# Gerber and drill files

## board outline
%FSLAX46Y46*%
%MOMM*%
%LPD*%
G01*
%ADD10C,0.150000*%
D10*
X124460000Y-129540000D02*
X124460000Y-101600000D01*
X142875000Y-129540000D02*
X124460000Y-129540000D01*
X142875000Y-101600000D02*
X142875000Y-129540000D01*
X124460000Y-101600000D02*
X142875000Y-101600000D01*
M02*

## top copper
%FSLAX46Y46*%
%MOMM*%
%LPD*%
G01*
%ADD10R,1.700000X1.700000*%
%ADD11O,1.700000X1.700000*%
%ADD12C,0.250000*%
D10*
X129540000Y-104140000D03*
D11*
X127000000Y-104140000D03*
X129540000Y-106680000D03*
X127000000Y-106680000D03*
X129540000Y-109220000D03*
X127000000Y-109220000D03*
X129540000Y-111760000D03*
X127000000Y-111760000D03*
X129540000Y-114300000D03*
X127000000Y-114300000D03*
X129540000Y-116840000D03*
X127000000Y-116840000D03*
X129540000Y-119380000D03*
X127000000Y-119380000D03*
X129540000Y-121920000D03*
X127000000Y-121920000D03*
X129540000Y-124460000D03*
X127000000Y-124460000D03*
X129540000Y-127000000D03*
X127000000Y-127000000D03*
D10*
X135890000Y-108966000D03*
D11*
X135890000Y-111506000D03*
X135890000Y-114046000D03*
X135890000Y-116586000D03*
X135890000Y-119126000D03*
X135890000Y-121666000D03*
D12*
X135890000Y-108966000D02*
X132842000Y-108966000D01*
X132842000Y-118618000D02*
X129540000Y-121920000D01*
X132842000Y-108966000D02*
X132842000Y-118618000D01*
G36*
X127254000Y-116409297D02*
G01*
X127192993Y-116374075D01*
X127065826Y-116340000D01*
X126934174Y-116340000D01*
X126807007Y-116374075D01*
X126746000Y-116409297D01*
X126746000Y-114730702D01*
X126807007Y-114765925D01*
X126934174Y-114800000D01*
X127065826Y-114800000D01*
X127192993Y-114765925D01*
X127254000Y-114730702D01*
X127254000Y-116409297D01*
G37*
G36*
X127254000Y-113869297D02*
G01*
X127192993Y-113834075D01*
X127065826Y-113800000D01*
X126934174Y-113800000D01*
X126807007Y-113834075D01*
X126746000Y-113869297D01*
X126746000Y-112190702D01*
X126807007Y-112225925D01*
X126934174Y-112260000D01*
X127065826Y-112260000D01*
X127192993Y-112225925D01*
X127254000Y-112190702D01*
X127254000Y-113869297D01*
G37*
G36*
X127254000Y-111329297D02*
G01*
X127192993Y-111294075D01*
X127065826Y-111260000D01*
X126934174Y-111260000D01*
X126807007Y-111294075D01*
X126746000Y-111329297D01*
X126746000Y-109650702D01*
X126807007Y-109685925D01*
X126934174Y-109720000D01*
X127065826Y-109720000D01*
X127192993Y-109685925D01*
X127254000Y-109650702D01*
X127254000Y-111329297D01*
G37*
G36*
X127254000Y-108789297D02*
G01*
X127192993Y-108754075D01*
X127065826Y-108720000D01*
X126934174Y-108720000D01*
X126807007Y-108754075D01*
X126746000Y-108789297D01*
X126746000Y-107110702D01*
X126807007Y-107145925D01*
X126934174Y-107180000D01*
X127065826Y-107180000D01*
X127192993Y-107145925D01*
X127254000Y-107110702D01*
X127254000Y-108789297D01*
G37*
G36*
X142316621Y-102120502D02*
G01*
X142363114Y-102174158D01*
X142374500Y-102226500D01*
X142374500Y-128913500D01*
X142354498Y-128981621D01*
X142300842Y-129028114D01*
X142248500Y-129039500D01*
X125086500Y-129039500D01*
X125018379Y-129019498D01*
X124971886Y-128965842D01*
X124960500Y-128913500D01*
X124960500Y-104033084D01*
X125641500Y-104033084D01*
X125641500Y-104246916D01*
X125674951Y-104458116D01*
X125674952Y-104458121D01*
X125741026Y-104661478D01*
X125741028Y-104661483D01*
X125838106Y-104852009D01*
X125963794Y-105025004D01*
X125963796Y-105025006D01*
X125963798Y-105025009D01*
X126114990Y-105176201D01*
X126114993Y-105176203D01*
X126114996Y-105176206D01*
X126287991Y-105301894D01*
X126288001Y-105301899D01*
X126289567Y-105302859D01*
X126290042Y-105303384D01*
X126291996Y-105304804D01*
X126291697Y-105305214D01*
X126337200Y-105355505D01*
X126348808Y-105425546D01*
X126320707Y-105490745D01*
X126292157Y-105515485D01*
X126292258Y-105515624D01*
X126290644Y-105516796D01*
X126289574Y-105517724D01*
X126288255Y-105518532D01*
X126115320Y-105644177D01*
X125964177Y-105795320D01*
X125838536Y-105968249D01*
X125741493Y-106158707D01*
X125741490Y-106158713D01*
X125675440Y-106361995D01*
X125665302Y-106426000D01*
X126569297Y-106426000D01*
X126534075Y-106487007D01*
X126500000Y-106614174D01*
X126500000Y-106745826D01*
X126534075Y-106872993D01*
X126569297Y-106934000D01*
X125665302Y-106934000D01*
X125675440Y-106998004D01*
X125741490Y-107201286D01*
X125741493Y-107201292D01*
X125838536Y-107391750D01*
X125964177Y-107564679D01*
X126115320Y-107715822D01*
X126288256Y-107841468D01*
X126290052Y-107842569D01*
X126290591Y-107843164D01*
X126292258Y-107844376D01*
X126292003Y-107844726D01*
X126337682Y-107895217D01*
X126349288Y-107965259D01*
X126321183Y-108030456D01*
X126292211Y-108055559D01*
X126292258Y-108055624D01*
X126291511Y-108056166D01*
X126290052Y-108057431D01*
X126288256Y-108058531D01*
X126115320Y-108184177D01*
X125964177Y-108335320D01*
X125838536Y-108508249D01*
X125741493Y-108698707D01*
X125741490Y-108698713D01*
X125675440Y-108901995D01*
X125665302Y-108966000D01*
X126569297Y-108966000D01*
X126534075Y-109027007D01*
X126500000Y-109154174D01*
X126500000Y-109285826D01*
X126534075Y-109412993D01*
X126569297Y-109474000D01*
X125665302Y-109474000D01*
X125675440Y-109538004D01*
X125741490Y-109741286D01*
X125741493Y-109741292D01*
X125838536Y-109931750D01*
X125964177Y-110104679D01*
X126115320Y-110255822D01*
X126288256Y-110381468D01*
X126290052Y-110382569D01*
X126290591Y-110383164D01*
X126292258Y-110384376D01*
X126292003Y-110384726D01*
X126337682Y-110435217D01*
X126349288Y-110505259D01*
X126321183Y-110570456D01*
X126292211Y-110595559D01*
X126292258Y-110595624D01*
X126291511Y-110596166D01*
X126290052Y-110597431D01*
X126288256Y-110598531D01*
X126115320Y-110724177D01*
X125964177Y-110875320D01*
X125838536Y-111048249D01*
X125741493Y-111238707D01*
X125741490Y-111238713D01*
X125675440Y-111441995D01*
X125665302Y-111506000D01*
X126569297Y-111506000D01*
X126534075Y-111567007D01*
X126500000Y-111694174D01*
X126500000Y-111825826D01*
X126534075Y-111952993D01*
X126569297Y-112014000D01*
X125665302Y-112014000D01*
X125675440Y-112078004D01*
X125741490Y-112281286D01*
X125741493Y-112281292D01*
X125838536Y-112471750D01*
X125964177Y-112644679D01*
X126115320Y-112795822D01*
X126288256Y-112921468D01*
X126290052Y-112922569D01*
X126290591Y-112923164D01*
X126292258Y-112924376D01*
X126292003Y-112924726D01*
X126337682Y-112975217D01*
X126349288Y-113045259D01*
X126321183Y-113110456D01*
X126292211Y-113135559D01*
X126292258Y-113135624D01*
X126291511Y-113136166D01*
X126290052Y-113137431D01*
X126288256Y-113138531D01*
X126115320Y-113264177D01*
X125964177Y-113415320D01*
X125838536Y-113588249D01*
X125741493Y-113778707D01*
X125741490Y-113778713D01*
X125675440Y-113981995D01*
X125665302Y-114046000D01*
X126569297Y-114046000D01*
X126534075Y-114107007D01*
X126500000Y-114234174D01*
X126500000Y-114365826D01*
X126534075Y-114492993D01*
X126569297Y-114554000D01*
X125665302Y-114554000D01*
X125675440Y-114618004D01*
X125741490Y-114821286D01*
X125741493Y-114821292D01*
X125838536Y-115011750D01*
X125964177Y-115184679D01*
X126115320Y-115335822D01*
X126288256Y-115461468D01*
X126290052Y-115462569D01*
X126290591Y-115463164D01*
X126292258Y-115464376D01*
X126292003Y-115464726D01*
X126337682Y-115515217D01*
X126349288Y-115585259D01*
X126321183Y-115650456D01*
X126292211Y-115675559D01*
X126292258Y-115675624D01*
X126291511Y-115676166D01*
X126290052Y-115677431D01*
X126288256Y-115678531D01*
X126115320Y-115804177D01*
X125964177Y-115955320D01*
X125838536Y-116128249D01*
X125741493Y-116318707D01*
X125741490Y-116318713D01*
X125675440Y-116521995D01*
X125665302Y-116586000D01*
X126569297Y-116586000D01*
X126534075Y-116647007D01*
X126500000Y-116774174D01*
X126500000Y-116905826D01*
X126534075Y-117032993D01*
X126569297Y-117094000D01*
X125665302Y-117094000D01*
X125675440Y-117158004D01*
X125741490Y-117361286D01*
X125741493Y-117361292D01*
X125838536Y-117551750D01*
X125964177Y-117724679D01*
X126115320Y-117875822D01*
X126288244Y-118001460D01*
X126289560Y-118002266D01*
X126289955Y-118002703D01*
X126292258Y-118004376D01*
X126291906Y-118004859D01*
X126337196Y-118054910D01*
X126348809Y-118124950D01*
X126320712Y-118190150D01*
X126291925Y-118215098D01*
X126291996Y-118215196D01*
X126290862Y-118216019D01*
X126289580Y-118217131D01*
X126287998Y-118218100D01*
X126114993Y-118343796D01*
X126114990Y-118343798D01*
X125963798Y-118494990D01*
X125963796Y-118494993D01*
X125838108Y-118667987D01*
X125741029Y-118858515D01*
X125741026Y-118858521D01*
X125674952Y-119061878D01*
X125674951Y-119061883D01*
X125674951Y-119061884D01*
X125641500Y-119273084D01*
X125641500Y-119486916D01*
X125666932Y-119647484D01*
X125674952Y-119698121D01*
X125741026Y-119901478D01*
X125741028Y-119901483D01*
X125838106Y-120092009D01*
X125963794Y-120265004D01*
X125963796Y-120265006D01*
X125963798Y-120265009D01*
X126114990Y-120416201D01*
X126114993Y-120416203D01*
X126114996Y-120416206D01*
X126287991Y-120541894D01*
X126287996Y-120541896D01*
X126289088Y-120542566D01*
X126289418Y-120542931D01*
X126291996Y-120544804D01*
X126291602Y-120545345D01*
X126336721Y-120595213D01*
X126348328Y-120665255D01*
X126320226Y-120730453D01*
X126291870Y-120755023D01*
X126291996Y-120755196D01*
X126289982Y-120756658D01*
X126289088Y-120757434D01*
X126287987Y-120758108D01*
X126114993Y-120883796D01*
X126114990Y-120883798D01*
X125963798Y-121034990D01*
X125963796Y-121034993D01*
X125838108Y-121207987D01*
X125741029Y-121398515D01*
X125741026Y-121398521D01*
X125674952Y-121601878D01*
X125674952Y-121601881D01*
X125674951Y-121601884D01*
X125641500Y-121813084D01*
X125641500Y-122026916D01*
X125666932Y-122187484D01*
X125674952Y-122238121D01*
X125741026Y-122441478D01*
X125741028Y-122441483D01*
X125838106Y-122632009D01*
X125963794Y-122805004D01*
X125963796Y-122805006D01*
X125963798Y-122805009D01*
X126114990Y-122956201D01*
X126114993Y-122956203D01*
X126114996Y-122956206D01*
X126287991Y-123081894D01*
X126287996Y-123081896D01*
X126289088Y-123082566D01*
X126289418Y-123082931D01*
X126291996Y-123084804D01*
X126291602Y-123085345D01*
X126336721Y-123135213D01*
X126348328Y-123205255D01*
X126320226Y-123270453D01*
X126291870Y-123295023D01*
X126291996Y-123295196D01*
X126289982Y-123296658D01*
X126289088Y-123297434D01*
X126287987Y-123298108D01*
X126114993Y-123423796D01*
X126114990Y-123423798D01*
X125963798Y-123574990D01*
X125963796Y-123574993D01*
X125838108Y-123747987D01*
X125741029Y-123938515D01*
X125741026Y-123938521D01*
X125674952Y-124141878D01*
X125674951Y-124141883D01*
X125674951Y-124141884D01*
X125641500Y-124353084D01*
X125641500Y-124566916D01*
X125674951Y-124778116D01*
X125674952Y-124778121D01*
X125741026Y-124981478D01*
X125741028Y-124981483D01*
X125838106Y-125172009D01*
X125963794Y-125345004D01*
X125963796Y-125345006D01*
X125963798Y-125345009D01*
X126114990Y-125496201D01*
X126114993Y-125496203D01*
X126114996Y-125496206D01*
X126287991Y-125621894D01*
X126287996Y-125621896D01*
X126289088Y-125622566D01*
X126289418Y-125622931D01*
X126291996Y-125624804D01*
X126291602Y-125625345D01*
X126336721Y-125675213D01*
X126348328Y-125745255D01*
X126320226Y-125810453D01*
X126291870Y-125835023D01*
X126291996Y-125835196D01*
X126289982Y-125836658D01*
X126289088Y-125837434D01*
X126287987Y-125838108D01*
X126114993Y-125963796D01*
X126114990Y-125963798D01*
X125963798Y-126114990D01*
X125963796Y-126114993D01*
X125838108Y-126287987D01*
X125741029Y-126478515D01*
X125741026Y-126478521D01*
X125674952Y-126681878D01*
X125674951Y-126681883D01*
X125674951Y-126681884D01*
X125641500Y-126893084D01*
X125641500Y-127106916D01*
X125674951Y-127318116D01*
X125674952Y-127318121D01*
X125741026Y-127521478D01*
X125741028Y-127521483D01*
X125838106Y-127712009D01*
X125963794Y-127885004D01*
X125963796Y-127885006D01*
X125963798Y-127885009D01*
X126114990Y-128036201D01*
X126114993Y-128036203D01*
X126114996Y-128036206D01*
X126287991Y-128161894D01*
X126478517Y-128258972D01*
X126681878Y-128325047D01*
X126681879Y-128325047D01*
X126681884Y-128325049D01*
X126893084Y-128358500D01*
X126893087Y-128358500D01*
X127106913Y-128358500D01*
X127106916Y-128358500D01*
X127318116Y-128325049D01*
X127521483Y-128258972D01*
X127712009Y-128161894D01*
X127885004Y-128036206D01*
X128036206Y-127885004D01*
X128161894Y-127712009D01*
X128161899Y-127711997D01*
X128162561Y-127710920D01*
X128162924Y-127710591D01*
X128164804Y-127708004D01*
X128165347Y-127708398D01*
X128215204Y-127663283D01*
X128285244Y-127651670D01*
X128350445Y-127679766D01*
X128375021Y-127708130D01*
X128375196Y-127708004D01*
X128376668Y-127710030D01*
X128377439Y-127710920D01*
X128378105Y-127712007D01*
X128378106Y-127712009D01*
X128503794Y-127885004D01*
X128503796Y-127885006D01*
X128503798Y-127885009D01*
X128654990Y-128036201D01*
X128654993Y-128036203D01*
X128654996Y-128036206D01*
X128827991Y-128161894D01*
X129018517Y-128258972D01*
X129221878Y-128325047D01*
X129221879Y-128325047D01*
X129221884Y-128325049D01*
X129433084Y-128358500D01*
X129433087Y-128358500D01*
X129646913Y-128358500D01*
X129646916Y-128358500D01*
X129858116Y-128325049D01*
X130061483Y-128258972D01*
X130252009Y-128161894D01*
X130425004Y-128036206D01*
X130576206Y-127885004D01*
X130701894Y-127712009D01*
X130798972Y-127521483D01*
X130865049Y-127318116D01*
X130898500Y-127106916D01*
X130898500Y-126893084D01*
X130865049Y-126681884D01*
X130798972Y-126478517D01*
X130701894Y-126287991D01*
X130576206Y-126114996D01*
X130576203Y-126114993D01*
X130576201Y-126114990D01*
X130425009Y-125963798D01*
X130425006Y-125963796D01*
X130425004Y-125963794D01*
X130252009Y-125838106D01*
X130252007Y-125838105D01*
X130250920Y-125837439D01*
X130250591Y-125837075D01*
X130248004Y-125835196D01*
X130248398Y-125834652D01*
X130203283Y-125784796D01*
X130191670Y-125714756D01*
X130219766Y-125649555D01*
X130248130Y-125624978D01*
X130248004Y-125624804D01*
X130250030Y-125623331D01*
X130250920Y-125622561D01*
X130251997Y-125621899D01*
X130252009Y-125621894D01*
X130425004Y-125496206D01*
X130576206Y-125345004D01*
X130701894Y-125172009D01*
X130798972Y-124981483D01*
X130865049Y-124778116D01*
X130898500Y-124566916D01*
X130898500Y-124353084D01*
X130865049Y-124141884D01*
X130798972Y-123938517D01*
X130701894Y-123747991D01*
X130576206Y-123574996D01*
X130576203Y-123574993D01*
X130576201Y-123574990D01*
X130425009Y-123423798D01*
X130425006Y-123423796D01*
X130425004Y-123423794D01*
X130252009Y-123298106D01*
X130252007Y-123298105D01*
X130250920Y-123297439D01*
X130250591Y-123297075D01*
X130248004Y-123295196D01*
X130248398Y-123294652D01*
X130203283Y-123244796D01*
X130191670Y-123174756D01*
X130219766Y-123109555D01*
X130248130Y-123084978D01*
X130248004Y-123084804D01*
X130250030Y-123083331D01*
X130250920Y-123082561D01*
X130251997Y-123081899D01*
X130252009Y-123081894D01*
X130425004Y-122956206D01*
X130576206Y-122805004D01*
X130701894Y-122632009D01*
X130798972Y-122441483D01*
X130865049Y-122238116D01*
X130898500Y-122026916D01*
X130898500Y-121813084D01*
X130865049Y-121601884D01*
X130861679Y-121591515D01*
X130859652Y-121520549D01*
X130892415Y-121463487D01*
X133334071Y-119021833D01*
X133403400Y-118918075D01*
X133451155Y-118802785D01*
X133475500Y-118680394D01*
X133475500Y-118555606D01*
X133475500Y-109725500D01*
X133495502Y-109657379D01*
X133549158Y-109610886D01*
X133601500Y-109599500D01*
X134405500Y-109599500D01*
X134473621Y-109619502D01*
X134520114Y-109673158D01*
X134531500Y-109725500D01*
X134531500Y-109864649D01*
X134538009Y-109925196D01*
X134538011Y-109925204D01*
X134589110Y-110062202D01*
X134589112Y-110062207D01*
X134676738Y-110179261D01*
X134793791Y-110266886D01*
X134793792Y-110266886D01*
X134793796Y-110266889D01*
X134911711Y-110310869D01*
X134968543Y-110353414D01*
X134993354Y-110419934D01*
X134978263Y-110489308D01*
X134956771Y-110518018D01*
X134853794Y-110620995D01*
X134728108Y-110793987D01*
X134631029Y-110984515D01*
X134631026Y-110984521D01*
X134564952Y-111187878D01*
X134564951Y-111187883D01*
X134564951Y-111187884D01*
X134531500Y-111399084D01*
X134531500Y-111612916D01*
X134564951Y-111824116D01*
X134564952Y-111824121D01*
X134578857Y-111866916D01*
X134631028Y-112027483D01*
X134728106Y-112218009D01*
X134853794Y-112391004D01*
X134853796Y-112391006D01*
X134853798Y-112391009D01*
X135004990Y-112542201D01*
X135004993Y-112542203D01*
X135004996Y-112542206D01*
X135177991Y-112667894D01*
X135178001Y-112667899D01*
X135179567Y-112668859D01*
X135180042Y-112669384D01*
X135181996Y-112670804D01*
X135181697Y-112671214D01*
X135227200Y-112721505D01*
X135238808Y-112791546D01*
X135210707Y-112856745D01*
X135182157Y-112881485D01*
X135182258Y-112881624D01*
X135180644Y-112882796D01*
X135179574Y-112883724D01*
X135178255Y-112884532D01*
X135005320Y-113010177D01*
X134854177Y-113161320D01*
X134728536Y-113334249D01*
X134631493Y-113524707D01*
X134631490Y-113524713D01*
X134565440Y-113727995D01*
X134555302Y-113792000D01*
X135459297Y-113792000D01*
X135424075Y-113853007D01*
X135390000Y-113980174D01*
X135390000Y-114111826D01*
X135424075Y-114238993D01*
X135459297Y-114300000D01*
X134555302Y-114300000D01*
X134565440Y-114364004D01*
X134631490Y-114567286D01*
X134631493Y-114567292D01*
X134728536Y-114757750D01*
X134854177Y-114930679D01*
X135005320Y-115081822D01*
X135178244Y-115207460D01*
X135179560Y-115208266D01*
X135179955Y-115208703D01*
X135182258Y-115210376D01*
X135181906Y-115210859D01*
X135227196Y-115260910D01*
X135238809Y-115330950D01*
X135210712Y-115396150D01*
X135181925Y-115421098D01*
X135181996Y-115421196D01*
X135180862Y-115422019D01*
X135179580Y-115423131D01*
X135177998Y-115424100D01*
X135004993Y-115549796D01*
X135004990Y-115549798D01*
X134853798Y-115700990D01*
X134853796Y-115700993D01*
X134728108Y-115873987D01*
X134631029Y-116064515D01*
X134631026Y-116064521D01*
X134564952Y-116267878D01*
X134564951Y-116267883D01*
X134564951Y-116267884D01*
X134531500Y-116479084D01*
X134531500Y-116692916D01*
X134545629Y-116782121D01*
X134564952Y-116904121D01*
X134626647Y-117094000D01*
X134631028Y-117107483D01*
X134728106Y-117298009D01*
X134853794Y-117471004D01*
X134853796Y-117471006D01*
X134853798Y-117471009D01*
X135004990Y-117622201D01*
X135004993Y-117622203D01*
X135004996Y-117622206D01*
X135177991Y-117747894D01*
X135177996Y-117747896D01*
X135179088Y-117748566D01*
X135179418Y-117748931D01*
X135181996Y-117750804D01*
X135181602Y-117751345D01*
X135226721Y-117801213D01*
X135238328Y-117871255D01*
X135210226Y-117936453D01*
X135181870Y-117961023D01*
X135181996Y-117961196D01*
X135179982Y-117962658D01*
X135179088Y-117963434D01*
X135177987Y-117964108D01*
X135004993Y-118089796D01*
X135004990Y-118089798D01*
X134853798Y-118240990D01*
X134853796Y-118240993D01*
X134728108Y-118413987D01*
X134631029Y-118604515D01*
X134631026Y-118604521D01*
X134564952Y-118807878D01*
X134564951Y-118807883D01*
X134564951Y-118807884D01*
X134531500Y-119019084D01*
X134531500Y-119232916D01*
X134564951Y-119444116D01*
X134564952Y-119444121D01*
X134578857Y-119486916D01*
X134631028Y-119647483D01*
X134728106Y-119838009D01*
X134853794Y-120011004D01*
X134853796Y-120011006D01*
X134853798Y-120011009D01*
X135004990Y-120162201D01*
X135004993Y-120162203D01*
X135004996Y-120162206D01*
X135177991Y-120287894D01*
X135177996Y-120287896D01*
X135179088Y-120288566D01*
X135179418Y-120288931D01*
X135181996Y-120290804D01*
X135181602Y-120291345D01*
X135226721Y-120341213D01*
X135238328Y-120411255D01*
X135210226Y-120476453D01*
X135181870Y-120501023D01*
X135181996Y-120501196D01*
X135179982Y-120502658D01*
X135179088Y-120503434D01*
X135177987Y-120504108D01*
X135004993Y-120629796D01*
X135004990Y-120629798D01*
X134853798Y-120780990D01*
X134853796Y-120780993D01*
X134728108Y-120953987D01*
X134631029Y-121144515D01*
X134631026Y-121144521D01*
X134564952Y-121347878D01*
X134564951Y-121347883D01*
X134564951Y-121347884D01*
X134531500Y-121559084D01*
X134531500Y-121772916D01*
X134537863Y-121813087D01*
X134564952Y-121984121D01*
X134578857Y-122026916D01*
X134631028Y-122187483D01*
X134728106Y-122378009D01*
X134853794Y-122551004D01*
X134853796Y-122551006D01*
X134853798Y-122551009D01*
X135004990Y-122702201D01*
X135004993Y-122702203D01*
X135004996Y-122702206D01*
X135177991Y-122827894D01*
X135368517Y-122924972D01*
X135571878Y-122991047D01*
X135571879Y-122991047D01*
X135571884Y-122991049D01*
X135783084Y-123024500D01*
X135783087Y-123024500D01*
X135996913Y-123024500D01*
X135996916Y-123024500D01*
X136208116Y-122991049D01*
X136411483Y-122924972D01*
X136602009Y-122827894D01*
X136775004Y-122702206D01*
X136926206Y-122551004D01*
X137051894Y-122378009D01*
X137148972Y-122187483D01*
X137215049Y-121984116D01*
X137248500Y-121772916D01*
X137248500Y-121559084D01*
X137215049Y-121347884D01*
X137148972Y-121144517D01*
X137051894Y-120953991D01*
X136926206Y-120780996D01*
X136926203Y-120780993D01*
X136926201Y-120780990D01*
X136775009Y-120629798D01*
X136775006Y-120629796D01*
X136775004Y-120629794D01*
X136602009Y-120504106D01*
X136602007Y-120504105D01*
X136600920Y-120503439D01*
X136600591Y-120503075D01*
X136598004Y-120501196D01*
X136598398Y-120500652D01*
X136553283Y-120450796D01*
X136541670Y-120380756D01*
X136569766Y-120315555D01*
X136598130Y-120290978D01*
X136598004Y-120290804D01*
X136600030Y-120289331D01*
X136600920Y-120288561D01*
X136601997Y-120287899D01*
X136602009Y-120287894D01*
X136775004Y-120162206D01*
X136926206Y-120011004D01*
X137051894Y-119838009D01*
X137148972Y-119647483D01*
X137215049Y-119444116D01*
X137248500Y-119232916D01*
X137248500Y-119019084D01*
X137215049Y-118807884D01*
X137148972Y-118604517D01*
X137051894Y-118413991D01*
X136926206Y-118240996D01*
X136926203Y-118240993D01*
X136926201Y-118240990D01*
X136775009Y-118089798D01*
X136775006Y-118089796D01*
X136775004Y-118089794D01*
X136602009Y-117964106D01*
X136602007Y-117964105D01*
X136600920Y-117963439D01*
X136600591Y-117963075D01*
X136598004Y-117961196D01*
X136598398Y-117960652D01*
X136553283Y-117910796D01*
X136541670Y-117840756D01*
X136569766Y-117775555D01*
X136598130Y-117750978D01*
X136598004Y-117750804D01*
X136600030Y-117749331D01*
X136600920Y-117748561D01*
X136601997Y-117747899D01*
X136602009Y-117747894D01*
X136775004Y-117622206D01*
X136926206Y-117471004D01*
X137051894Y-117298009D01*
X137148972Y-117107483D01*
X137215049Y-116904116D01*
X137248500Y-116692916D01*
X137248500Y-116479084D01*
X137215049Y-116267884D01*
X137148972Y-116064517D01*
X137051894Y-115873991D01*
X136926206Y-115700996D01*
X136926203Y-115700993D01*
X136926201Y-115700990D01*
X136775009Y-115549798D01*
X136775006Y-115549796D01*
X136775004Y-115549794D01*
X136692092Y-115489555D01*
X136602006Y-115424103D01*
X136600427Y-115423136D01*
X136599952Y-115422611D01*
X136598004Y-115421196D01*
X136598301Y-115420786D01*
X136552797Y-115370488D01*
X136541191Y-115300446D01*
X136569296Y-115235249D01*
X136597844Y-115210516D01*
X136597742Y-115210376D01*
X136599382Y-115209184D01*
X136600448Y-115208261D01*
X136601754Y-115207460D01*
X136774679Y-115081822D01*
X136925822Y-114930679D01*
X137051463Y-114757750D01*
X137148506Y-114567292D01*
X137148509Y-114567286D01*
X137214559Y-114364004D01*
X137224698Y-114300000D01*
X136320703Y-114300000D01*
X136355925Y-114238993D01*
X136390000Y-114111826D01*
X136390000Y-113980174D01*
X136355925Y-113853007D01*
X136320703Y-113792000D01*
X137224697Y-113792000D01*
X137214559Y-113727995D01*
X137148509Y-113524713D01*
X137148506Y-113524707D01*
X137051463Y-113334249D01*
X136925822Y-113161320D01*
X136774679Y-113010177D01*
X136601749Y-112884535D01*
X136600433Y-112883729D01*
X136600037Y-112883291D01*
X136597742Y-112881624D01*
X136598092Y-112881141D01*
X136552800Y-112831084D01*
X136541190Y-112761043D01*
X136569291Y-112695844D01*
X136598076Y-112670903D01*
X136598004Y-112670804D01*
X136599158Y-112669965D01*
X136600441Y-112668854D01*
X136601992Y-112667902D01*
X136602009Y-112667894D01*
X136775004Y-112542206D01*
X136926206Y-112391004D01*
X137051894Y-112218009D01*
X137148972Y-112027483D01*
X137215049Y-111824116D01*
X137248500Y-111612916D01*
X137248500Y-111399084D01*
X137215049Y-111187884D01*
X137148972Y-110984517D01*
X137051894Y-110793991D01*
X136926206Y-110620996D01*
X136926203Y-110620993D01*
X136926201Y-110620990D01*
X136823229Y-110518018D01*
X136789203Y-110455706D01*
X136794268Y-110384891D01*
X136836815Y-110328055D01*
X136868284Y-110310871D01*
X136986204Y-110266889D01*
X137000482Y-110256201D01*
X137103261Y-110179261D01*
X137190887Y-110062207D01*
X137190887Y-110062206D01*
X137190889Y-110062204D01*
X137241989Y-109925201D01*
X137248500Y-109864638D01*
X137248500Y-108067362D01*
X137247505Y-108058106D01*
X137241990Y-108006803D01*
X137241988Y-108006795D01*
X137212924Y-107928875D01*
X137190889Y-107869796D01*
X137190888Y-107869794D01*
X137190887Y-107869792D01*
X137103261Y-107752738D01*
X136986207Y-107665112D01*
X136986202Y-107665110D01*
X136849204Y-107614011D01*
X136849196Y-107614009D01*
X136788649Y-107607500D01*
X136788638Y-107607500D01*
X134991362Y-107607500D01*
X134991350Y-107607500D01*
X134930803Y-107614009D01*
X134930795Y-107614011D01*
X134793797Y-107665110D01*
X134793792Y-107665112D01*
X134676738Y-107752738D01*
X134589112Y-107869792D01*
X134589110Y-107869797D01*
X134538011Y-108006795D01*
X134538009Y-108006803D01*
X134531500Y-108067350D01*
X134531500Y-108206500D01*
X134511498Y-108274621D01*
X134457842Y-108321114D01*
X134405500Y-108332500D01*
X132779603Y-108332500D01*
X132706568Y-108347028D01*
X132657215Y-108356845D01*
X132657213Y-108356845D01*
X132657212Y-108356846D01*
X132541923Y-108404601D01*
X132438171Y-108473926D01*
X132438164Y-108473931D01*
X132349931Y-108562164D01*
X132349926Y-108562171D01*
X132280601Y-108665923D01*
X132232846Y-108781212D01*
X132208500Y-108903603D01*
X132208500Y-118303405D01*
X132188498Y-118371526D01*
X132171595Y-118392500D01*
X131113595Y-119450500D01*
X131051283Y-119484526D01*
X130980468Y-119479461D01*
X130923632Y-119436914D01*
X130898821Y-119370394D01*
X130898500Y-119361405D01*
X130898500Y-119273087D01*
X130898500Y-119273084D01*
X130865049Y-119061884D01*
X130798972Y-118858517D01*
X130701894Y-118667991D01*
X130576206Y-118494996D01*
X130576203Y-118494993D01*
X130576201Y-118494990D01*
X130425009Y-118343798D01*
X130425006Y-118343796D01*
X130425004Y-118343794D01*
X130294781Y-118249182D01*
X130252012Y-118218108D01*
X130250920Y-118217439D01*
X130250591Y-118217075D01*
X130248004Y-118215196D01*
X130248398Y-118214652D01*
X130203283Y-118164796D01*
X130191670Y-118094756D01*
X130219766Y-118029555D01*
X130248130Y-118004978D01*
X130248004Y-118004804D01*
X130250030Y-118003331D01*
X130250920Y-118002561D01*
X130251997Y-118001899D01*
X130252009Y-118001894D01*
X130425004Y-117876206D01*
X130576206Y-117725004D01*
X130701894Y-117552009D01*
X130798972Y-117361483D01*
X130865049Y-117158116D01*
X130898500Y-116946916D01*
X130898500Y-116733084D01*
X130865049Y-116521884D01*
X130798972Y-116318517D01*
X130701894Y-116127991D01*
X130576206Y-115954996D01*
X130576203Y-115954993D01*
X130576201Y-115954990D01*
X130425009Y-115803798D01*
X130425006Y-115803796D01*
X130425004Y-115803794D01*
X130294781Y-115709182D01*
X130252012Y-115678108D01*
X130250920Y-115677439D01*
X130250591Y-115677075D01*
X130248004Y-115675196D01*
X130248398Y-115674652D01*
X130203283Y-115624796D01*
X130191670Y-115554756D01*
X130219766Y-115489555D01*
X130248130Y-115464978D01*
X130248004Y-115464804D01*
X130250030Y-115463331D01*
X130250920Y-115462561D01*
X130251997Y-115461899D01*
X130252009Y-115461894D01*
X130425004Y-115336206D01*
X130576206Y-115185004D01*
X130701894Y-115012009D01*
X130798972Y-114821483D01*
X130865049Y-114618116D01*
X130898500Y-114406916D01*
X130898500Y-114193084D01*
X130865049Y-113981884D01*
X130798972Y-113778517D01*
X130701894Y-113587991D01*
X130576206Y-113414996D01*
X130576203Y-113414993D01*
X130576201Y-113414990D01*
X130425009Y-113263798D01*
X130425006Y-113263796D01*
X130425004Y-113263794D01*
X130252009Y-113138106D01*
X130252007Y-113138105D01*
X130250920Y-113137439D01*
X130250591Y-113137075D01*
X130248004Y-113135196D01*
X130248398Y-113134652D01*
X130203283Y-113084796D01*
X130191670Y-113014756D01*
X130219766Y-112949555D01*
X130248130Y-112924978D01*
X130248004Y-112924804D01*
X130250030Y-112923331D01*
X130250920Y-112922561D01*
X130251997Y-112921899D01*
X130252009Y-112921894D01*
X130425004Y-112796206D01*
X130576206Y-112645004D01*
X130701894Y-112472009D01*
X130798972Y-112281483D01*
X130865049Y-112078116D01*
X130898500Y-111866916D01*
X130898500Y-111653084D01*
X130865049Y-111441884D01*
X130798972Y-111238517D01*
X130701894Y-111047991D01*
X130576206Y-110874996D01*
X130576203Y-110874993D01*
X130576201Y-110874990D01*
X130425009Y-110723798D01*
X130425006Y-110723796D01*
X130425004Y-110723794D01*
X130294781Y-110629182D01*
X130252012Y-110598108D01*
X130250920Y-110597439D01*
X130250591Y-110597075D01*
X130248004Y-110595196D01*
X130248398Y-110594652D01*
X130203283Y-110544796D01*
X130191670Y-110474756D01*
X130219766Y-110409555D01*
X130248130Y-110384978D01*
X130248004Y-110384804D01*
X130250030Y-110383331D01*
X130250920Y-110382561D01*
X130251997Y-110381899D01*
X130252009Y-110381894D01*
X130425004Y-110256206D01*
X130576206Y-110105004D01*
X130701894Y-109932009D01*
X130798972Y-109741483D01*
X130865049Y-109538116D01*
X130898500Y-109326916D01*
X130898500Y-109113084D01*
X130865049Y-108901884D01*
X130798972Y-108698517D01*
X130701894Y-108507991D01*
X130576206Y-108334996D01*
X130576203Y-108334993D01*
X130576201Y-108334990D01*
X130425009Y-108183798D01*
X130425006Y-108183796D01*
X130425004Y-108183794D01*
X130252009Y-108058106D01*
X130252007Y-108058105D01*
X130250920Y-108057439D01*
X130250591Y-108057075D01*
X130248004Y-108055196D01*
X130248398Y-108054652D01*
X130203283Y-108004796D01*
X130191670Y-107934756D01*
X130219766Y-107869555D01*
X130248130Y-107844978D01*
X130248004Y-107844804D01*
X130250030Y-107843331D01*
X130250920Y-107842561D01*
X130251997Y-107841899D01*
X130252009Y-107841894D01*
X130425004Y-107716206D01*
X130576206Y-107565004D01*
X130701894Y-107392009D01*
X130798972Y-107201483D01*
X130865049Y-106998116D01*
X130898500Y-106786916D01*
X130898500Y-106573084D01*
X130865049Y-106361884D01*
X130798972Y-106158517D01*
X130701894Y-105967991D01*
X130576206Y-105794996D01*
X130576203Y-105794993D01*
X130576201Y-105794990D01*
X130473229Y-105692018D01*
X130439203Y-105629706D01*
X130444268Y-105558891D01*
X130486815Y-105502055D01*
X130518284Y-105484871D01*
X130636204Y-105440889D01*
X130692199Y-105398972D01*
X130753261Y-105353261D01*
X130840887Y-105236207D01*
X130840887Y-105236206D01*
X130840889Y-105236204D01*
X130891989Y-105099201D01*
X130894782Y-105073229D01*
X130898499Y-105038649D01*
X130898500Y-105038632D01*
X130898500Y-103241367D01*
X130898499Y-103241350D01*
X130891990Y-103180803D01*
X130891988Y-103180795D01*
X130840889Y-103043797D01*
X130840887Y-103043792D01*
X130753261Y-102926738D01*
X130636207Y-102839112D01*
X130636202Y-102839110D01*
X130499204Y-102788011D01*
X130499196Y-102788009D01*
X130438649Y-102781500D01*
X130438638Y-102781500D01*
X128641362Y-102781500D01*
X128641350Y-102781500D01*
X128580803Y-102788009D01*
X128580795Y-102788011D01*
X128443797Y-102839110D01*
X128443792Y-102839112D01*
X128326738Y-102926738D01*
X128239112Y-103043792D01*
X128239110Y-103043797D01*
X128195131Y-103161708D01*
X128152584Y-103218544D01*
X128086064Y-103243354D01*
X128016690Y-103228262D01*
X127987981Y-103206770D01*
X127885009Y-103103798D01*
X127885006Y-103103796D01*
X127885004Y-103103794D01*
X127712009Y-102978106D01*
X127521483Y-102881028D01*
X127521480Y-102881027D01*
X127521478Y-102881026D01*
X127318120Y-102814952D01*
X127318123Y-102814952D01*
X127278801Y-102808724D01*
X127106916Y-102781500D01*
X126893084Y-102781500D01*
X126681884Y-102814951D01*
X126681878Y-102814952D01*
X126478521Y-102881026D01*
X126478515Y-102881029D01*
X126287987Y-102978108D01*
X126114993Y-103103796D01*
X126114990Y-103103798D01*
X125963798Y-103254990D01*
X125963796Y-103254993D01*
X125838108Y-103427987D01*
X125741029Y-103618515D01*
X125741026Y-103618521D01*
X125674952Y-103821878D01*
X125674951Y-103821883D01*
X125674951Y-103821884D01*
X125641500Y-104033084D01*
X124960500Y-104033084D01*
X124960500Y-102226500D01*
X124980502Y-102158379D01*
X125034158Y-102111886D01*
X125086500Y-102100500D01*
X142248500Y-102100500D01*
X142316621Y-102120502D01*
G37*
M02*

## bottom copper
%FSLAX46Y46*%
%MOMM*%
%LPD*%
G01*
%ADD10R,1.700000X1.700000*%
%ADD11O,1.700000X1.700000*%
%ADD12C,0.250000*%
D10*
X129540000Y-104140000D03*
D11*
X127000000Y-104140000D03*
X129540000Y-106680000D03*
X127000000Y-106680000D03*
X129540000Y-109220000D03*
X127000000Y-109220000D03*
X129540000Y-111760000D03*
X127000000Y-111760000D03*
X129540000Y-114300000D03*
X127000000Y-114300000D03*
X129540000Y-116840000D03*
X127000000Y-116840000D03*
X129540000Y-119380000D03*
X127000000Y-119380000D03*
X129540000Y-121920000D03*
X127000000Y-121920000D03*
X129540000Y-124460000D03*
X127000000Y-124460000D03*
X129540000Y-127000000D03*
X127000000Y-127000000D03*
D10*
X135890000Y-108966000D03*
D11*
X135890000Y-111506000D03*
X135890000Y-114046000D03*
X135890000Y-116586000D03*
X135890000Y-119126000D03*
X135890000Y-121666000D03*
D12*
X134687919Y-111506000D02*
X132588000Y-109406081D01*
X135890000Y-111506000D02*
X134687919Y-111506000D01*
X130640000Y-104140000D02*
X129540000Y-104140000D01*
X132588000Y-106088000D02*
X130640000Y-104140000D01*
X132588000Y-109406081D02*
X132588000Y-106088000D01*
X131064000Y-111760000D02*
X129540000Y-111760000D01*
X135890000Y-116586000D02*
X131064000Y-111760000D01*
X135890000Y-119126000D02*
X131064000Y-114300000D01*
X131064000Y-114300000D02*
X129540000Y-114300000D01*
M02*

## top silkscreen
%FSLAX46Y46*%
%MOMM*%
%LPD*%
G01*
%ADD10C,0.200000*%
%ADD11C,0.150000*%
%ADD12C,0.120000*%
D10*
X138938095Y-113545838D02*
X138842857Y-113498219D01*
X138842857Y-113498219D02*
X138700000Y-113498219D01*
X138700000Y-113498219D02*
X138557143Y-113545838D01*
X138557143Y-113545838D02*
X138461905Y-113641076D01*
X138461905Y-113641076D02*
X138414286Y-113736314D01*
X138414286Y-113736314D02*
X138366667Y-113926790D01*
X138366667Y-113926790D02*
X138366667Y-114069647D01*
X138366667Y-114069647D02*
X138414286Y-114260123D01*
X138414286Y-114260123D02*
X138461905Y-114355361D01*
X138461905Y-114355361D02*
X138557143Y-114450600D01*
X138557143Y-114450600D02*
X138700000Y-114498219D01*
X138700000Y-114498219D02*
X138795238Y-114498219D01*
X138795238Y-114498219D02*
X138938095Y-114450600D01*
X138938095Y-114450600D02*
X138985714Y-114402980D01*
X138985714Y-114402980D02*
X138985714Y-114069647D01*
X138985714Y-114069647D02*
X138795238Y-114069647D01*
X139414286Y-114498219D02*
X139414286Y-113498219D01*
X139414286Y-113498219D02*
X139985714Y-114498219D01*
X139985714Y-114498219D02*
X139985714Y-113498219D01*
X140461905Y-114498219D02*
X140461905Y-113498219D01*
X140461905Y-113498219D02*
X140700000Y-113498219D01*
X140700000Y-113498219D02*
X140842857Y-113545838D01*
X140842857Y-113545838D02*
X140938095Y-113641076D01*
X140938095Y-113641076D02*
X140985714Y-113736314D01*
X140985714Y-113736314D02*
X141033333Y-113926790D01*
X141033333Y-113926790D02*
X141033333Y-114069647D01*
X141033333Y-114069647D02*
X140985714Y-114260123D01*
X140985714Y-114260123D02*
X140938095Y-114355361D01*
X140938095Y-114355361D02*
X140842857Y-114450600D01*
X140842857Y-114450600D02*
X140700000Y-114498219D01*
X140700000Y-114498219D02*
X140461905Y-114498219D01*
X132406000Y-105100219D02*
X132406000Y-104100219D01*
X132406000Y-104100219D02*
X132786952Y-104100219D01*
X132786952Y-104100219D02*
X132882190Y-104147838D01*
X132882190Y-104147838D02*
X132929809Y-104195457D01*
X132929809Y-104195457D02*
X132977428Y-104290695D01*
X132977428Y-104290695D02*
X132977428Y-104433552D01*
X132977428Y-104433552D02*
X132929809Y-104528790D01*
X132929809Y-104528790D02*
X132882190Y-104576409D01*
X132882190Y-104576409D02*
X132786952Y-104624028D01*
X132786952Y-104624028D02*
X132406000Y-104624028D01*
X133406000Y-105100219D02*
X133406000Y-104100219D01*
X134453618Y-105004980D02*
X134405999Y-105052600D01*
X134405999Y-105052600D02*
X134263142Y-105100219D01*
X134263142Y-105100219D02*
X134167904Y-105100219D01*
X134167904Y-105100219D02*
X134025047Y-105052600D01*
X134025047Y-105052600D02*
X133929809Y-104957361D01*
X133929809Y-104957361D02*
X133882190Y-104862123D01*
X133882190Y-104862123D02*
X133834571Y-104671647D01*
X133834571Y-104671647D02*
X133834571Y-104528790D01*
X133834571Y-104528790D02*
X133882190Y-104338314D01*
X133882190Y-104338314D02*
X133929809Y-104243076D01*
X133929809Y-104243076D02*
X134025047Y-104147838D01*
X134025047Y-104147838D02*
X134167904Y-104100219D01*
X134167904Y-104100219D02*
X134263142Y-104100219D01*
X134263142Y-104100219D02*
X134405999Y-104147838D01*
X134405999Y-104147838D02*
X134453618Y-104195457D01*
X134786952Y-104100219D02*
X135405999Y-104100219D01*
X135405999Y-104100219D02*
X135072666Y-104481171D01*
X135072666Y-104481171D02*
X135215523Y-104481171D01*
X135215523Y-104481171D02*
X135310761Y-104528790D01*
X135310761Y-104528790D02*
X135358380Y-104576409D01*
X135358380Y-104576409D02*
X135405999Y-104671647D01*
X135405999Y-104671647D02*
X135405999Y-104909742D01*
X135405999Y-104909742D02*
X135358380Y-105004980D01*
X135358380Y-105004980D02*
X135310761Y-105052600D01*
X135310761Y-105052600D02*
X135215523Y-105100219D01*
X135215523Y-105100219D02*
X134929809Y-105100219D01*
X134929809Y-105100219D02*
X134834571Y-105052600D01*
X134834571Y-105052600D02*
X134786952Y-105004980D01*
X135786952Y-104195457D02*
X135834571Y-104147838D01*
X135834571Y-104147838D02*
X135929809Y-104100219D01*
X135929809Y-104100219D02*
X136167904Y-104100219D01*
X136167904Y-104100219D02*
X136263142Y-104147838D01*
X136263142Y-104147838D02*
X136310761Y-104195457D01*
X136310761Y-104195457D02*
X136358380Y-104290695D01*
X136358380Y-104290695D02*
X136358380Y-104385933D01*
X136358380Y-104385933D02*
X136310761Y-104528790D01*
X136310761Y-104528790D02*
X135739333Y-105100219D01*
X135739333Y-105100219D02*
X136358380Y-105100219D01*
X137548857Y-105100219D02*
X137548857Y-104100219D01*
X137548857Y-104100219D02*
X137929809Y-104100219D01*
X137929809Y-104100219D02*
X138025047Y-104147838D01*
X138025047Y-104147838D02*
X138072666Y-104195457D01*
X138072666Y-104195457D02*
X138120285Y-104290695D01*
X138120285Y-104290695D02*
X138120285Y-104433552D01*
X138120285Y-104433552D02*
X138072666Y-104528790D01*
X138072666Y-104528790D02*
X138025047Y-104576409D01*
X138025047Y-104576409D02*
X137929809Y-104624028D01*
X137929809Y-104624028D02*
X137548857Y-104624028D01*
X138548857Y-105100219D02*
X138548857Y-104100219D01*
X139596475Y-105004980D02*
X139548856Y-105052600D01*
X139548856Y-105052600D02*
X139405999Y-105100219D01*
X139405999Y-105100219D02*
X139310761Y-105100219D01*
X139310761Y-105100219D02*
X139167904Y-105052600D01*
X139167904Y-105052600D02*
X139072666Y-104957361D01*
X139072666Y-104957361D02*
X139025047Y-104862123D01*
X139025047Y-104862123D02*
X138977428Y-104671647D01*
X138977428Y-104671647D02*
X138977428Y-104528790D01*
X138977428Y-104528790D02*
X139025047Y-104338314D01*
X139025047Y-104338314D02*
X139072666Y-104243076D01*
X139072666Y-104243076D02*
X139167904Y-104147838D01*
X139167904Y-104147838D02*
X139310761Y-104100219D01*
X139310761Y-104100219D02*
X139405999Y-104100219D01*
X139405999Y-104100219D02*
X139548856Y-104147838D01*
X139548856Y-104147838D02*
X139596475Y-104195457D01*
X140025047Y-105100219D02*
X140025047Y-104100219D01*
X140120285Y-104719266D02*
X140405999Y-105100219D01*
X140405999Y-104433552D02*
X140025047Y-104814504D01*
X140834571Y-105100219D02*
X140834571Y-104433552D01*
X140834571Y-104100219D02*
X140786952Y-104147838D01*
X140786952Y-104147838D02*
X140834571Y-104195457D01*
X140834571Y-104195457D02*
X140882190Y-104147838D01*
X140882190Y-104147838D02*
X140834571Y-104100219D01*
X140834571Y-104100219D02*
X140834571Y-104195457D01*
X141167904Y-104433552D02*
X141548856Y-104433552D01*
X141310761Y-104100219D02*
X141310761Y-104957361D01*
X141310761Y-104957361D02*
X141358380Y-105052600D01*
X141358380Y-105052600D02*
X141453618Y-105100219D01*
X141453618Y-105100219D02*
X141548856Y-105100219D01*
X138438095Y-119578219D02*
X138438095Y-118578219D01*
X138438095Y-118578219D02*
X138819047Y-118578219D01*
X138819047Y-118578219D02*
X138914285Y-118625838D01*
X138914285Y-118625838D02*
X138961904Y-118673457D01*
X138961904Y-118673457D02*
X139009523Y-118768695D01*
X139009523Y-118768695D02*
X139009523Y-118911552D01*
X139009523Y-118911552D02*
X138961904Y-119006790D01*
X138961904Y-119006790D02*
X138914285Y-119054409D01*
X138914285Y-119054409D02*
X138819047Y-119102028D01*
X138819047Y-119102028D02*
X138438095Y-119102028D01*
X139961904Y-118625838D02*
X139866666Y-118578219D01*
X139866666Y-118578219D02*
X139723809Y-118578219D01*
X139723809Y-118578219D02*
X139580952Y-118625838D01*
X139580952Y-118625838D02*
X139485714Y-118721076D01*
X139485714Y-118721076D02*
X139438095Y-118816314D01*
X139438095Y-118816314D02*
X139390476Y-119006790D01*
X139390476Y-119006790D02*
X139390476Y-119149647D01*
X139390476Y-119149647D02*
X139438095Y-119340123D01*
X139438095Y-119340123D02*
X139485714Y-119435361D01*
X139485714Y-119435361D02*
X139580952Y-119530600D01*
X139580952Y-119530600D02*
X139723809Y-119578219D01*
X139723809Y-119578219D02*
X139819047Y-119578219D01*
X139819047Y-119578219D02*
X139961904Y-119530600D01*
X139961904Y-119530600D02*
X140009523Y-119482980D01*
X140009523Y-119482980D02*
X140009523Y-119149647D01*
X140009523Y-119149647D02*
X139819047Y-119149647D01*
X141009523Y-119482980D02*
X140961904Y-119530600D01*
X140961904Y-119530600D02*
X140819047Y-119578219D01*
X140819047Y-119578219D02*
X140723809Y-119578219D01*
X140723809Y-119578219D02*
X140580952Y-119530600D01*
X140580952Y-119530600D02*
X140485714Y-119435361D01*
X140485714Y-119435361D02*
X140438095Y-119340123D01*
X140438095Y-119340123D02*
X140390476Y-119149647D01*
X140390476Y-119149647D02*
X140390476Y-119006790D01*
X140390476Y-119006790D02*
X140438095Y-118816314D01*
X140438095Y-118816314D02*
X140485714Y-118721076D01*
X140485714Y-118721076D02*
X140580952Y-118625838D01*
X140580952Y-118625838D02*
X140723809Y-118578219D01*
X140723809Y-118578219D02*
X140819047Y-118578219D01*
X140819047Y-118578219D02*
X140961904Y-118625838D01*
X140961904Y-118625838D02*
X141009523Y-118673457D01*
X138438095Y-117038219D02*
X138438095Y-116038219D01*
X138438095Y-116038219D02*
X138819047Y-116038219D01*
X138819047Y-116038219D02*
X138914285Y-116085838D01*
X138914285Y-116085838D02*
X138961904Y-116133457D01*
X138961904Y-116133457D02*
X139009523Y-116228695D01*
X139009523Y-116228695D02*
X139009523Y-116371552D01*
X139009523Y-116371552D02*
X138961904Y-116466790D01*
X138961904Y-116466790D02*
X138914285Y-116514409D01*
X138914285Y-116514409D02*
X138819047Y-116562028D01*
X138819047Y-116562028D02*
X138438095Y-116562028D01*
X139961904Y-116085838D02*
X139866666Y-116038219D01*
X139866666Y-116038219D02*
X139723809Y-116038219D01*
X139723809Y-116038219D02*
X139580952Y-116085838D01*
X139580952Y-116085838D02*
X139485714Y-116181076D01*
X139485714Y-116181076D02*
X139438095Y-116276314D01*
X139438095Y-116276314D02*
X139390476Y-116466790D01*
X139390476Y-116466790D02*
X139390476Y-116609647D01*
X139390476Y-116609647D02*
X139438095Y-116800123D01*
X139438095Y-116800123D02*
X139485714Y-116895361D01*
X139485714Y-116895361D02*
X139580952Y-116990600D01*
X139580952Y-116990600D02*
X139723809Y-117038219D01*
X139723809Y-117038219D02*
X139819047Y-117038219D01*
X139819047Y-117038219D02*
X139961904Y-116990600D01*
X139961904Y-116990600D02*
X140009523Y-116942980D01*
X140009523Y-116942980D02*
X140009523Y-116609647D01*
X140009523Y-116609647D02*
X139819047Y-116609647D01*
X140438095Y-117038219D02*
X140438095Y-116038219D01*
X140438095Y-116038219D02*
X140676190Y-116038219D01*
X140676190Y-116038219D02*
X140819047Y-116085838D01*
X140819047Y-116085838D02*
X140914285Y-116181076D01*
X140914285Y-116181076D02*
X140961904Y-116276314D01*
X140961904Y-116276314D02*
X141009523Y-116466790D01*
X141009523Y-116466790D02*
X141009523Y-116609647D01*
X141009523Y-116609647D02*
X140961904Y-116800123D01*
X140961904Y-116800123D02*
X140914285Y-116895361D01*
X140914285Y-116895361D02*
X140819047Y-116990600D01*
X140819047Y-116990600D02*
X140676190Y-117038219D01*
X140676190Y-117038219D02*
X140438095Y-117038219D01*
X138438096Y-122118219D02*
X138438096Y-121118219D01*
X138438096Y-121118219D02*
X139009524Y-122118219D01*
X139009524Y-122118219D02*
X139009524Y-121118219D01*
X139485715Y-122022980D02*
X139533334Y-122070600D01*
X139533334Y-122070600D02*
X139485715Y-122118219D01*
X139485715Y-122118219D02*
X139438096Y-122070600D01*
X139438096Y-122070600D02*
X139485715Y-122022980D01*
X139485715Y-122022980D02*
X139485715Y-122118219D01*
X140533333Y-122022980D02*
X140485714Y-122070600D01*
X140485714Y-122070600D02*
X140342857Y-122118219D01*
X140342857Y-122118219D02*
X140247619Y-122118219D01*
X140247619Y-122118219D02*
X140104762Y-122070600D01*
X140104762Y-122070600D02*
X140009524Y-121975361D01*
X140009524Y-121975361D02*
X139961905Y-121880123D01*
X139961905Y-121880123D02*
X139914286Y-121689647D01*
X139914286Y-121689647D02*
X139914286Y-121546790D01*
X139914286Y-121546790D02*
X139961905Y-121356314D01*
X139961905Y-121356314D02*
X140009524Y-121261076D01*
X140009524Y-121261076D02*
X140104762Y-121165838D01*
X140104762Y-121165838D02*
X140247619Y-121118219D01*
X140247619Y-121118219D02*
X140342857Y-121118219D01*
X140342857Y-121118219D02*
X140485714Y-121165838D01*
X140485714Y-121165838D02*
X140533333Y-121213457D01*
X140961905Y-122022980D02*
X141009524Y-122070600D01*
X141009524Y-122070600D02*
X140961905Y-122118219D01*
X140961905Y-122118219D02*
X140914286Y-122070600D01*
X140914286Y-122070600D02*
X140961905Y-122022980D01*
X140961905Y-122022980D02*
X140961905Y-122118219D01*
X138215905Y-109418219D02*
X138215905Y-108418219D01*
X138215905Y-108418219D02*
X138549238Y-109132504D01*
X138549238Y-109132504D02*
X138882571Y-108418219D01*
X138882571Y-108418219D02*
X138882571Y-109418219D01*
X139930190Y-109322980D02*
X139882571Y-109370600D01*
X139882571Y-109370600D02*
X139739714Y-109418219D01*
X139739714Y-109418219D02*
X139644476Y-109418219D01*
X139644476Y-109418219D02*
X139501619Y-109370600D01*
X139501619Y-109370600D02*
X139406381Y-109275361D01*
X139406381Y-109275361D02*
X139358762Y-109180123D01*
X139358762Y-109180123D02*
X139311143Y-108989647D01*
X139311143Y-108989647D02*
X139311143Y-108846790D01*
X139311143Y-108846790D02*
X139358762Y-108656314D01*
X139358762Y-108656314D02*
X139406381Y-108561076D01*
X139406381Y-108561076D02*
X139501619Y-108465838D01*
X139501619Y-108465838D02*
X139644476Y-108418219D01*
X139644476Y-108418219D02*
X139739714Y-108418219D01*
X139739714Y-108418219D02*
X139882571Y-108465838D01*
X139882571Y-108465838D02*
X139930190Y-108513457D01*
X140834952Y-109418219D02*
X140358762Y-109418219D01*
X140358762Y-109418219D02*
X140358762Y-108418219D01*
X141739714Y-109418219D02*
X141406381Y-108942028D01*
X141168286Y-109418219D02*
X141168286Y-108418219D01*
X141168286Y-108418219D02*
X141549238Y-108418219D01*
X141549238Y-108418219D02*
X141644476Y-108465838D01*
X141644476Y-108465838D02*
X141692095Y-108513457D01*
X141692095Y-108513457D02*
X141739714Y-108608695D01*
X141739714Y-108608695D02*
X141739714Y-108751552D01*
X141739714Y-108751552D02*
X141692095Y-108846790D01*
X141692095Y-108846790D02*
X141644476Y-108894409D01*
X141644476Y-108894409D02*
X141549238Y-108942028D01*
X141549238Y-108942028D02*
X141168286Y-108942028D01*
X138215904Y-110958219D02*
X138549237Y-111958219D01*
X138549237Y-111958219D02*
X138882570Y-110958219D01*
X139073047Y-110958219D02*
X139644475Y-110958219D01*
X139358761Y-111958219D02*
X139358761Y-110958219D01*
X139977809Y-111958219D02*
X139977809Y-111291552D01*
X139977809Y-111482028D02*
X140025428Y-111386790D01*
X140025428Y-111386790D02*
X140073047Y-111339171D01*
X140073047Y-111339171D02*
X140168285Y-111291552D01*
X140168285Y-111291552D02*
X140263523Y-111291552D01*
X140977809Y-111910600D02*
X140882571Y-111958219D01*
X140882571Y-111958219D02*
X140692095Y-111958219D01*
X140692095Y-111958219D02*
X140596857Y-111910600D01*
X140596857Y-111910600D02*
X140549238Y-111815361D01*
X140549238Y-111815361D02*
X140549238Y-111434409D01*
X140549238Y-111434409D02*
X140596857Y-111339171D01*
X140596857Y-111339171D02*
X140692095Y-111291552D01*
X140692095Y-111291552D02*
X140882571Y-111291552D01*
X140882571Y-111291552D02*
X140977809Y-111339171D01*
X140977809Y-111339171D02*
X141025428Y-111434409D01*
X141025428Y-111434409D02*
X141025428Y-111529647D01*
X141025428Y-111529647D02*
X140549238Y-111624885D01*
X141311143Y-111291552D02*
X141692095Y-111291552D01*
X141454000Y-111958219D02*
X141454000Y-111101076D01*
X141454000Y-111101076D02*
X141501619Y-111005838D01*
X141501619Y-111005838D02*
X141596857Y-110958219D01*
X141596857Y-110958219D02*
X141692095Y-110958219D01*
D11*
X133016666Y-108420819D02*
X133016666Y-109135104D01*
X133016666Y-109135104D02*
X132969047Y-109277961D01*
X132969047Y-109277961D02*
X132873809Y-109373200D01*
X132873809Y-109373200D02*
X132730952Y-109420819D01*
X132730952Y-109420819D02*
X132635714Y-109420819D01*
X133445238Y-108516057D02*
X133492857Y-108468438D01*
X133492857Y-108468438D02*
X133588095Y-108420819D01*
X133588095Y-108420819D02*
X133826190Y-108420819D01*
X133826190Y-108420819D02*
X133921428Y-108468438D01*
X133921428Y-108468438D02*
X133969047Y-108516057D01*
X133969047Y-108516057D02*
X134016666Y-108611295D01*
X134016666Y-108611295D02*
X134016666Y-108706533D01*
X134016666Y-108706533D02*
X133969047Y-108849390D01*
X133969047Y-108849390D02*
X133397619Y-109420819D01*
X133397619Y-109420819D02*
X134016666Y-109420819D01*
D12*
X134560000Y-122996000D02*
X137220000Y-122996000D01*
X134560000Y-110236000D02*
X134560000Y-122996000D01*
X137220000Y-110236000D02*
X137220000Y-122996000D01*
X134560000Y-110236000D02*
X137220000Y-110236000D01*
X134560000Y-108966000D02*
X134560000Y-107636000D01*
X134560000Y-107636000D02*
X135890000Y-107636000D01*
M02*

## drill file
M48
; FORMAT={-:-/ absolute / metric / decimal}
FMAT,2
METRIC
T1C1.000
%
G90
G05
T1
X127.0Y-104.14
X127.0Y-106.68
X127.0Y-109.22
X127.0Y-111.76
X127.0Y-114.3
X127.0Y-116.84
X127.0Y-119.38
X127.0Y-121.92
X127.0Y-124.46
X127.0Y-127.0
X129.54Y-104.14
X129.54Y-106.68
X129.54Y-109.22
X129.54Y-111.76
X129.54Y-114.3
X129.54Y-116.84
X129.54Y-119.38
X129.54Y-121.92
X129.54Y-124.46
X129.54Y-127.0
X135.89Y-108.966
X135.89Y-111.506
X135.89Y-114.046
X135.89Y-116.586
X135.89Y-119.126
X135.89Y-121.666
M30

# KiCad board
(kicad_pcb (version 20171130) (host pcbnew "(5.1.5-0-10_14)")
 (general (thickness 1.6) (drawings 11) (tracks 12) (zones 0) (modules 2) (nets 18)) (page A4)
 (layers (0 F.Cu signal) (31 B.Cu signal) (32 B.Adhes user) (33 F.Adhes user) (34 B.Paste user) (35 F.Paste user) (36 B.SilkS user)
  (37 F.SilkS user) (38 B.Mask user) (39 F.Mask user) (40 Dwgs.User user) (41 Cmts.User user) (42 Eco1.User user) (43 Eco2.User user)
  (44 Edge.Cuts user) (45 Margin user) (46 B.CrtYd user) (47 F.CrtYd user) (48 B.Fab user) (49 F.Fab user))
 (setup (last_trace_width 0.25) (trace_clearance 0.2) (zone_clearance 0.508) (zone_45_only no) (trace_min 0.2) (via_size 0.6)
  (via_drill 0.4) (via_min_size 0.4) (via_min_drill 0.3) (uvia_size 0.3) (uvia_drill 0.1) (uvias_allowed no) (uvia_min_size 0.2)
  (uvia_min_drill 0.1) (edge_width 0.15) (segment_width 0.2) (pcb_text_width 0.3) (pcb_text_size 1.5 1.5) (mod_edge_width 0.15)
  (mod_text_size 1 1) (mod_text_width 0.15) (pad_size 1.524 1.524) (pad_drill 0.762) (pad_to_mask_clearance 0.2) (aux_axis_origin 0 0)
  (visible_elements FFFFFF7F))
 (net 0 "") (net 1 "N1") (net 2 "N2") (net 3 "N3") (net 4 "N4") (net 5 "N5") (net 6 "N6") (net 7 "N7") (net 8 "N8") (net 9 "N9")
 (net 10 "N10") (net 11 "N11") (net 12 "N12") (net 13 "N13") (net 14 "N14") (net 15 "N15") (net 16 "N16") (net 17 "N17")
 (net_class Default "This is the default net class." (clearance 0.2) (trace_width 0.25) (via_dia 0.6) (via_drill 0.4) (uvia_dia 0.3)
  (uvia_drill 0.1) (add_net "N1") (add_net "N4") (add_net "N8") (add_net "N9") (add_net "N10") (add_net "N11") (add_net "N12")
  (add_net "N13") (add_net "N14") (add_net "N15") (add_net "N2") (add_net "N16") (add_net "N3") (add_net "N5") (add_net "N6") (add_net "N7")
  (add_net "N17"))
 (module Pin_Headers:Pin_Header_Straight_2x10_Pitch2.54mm (layer B.Cu) (at 129.54 104.14 180)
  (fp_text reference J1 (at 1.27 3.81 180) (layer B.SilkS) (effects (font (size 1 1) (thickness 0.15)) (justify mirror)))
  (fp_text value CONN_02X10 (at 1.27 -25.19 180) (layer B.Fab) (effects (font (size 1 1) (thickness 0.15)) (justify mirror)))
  (pad 1 thru_hole rect (at 0 0 180) (size 1.7 1.7) (drill 1) (layers *.Cu *.Mask) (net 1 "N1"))
  (pad 2 thru_hole oval (at 2.54 0 180) (size 1.7 1.7) (drill 1) (layers *.Cu *.Mask) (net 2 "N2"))
  (pad 3 thru_hole oval (at 0 -2.54 180) (size 1.7 1.7) (drill 1) (layers *.Cu *.Mask) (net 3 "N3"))
  (pad 4 thru_hole oval (at 2.54 -2.54 180) (size 1.7 1.7) (drill 1) (layers *.Cu *.Mask) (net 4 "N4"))
  (pad 5 thru_hole oval (at 0 -5.08 180) (size 1.7 1.7) (drill 1) (layers *.Cu *.Mask) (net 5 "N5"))
  (pad 6 thru_hole oval (at 2.54 -5.08 180) (size 1.7 1.7) (drill 1) (layers *.Cu *.Mask) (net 4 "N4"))
  (pad 7 thru_hole oval (at 0 -7.62 180) (size 1.7 1.7) (drill 1) (layers *.Cu *.Mask) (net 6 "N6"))
  (pad 8 thru_hole oval (at 2.54 -7.62 180) (size 1.7 1.7) (drill 1) (layers *.Cu *.Mask) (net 4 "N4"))
  (pad 9 thru_hole oval (at 0 -10.16 180) (size 1.7 1.7) (drill 1) (layers *.Cu *.Mask) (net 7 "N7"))
  (pad 10 thru_hole oval (at 2.54 -10.16 180) (size 1.7 1.7) (drill 1) (layers *.Cu *.Mask) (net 4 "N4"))
  (pad 11 thru_hole oval (at 0 -12.7 180) (size 1.7 1.7) (drill 1) (layers *.Cu *.Mask) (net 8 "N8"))
  (pad 12 thru_hole oval (at 2.54 -12.7 180) (size 1.7 1.7) (drill 1) (layers *.Cu *.Mask) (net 4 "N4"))
  (pad 13 thru_hole oval (at 0 -15.24 180) (size 1.7 1.7) (drill 1) (layers *.Cu *.Mask) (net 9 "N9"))
  (pad 14 thru_hole oval (at 2.54 -15.24 180) (size 1.7 1.7) (drill 1) (layers *.Cu *.Mask) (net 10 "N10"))
  (pad 15 thru_hole oval (at 0 -17.78 180) (size 1.7 1.7) (drill 1) (layers *.Cu *.Mask) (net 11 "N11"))
  (pad 16 thru_hole oval (at 2.54 -17.78 180) (size 1.7 1.7) (drill 1) (layers *.Cu *.Mask) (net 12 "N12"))
  (pad 17 thru_hole oval (at 0 -20.32 180) (size 1.7 1.7) (drill 1) (layers *.Cu *.Mask) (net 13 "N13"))
  (pad 18 thru_hole oval (at 2.54 -20.32 180) (size 1.7 1.7) (drill 1) (layers *.Cu *.Mask) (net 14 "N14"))
  (pad 19 thru_hole oval (at 0 -22.86 180) (size 1.7 1.7) (drill 1) (layers *.Cu *.Mask) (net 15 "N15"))
  (pad 20 thru_hole oval (at 2.54 -22.86 180) (size 1.7 1.7) (drill 1) (layers *.Cu *.Mask) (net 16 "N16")))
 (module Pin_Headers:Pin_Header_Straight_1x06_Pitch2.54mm (layer F.Cu) (at 135.89 108.966)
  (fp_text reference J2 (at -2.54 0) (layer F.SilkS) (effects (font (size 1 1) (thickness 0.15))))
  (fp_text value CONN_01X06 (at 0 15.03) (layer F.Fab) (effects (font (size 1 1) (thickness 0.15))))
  (fp_line (start -1.33 14.03) (end 1.33 14.03) (layer F.SilkS) (width 0.12))
  (fp_line (start -1.33 1.27) (end -1.33 14.03) (layer F.SilkS) (width 0.12))
  (fp_line (start 1.33 1.27) (end 1.33 14.03) (layer F.SilkS) (width 0.12))
  (fp_line (start -1.33 1.27) (end 1.33 1.27) (layer F.SilkS) (width 0.12))
  (fp_line (start -1.33 0) (end -1.33 -1.33) (layer F.SilkS) (width 0.12))
  (fp_line (start -1.33 -1.33) (end 0 -1.33) (layer F.SilkS) (width 0.12))
  (pad 1 thru_hole rect (at 0 0) (size 1.7 1.7) (drill 1) (layers *.Cu *.Mask) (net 11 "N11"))
  (pad 2 thru_hole oval (at 0 2.54) (size 1.7 1.7) (drill 1) (layers *.Cu *.Mask) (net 1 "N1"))
  (pad 3 thru_hole oval (at 0 5.08) (size 1.7 1.7) (drill 1) (layers *.Cu *.Mask) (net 4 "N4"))
  (pad 4 thru_hole oval (at 0 7.62) (size 1.7 1.7) (drill 1) (layers *.Cu *.Mask) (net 6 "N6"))
  (pad 5 thru_hole oval (at 0 10.16) (size 1.7 1.7) (drill 1) (layers *.Cu *.Mask) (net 7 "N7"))
  (pad 6 thru_hole oval (at 0 12.7) (size 1.7 1.7) (drill 1) (layers *.Cu *.Mask) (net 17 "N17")))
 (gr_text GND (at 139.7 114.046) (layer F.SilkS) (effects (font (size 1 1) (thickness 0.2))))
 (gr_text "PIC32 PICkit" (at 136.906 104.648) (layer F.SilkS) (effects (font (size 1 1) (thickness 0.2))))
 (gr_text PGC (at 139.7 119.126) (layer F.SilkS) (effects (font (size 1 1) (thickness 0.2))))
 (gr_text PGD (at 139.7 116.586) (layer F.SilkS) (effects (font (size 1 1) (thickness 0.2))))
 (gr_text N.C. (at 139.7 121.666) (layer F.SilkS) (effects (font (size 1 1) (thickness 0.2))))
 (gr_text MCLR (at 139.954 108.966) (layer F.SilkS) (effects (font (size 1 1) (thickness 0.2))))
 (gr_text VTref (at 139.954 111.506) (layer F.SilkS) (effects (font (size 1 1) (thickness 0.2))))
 (gr_line (start 124.46 129.54) (end 124.46 101.6) (angle 90) (layer Edge.Cuts) (width 0.15))
 (gr_line (start 142.875 129.54) (end 124.46 129.54) (angle 90) (layer Edge.Cuts) (width 0.15))
 (gr_line (start 142.875 101.6) (end 142.875 129.54) (angle 90) (layer Edge.Cuts) (width 0.15))
 (gr_line (start 124.46 101.6) (end 142.875 101.6) (angle 90) (layer Edge.Cuts) (width 0.15))
 (segment (start 134.687919 111.506) (end 132.588 109.406081) (width 0.25) (layer B.Cu) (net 1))
 (segment (start 135.89 111.506) (end 134.687919 111.506) (width 0.25) (layer B.Cu) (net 1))
 (segment (start 130.64 104.14) (end 129.54 104.14) (width 0.25) (layer B.Cu) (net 1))
 (segment (start 132.588 106.088) (end 130.64 104.14) (width 0.25) (layer B.Cu) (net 1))
 (segment (start 132.588 109.406081) (end 132.588 106.088) (width 0.25) (layer B.Cu) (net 1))
 (segment (start 131.064 111.76) (end 129.54 111.76) (width 0.25) (layer B.Cu) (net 6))
 (segment (start 135.89 116.586) (end 131.064 111.76) (width 0.25) (layer B.Cu) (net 6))
 (segment (start 135.89 119.126) (end 131.064 114.3) (width 0.25) (layer B.Cu) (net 7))
 (segment (start 131.064 114.3) (end 129.54 114.3) (width 0.25) (layer B.Cu) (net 7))
 (segment (start 135.89 108.966) (end 132.842 108.966) (width 0.25) (layer F.Cu) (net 11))
 (segment (start 132.842 118.618) (end 129.54 121.92) (width 0.25) (layer F.Cu) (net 11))
 (segment (start 132.842 108.966) (end 132.842 118.618) (width 0.25) (layer F.Cu) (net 11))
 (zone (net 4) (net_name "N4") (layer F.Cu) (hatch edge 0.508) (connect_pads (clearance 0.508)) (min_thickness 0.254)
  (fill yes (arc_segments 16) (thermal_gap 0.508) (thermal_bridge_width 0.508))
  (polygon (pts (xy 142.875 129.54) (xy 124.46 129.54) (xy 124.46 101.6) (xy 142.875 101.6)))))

